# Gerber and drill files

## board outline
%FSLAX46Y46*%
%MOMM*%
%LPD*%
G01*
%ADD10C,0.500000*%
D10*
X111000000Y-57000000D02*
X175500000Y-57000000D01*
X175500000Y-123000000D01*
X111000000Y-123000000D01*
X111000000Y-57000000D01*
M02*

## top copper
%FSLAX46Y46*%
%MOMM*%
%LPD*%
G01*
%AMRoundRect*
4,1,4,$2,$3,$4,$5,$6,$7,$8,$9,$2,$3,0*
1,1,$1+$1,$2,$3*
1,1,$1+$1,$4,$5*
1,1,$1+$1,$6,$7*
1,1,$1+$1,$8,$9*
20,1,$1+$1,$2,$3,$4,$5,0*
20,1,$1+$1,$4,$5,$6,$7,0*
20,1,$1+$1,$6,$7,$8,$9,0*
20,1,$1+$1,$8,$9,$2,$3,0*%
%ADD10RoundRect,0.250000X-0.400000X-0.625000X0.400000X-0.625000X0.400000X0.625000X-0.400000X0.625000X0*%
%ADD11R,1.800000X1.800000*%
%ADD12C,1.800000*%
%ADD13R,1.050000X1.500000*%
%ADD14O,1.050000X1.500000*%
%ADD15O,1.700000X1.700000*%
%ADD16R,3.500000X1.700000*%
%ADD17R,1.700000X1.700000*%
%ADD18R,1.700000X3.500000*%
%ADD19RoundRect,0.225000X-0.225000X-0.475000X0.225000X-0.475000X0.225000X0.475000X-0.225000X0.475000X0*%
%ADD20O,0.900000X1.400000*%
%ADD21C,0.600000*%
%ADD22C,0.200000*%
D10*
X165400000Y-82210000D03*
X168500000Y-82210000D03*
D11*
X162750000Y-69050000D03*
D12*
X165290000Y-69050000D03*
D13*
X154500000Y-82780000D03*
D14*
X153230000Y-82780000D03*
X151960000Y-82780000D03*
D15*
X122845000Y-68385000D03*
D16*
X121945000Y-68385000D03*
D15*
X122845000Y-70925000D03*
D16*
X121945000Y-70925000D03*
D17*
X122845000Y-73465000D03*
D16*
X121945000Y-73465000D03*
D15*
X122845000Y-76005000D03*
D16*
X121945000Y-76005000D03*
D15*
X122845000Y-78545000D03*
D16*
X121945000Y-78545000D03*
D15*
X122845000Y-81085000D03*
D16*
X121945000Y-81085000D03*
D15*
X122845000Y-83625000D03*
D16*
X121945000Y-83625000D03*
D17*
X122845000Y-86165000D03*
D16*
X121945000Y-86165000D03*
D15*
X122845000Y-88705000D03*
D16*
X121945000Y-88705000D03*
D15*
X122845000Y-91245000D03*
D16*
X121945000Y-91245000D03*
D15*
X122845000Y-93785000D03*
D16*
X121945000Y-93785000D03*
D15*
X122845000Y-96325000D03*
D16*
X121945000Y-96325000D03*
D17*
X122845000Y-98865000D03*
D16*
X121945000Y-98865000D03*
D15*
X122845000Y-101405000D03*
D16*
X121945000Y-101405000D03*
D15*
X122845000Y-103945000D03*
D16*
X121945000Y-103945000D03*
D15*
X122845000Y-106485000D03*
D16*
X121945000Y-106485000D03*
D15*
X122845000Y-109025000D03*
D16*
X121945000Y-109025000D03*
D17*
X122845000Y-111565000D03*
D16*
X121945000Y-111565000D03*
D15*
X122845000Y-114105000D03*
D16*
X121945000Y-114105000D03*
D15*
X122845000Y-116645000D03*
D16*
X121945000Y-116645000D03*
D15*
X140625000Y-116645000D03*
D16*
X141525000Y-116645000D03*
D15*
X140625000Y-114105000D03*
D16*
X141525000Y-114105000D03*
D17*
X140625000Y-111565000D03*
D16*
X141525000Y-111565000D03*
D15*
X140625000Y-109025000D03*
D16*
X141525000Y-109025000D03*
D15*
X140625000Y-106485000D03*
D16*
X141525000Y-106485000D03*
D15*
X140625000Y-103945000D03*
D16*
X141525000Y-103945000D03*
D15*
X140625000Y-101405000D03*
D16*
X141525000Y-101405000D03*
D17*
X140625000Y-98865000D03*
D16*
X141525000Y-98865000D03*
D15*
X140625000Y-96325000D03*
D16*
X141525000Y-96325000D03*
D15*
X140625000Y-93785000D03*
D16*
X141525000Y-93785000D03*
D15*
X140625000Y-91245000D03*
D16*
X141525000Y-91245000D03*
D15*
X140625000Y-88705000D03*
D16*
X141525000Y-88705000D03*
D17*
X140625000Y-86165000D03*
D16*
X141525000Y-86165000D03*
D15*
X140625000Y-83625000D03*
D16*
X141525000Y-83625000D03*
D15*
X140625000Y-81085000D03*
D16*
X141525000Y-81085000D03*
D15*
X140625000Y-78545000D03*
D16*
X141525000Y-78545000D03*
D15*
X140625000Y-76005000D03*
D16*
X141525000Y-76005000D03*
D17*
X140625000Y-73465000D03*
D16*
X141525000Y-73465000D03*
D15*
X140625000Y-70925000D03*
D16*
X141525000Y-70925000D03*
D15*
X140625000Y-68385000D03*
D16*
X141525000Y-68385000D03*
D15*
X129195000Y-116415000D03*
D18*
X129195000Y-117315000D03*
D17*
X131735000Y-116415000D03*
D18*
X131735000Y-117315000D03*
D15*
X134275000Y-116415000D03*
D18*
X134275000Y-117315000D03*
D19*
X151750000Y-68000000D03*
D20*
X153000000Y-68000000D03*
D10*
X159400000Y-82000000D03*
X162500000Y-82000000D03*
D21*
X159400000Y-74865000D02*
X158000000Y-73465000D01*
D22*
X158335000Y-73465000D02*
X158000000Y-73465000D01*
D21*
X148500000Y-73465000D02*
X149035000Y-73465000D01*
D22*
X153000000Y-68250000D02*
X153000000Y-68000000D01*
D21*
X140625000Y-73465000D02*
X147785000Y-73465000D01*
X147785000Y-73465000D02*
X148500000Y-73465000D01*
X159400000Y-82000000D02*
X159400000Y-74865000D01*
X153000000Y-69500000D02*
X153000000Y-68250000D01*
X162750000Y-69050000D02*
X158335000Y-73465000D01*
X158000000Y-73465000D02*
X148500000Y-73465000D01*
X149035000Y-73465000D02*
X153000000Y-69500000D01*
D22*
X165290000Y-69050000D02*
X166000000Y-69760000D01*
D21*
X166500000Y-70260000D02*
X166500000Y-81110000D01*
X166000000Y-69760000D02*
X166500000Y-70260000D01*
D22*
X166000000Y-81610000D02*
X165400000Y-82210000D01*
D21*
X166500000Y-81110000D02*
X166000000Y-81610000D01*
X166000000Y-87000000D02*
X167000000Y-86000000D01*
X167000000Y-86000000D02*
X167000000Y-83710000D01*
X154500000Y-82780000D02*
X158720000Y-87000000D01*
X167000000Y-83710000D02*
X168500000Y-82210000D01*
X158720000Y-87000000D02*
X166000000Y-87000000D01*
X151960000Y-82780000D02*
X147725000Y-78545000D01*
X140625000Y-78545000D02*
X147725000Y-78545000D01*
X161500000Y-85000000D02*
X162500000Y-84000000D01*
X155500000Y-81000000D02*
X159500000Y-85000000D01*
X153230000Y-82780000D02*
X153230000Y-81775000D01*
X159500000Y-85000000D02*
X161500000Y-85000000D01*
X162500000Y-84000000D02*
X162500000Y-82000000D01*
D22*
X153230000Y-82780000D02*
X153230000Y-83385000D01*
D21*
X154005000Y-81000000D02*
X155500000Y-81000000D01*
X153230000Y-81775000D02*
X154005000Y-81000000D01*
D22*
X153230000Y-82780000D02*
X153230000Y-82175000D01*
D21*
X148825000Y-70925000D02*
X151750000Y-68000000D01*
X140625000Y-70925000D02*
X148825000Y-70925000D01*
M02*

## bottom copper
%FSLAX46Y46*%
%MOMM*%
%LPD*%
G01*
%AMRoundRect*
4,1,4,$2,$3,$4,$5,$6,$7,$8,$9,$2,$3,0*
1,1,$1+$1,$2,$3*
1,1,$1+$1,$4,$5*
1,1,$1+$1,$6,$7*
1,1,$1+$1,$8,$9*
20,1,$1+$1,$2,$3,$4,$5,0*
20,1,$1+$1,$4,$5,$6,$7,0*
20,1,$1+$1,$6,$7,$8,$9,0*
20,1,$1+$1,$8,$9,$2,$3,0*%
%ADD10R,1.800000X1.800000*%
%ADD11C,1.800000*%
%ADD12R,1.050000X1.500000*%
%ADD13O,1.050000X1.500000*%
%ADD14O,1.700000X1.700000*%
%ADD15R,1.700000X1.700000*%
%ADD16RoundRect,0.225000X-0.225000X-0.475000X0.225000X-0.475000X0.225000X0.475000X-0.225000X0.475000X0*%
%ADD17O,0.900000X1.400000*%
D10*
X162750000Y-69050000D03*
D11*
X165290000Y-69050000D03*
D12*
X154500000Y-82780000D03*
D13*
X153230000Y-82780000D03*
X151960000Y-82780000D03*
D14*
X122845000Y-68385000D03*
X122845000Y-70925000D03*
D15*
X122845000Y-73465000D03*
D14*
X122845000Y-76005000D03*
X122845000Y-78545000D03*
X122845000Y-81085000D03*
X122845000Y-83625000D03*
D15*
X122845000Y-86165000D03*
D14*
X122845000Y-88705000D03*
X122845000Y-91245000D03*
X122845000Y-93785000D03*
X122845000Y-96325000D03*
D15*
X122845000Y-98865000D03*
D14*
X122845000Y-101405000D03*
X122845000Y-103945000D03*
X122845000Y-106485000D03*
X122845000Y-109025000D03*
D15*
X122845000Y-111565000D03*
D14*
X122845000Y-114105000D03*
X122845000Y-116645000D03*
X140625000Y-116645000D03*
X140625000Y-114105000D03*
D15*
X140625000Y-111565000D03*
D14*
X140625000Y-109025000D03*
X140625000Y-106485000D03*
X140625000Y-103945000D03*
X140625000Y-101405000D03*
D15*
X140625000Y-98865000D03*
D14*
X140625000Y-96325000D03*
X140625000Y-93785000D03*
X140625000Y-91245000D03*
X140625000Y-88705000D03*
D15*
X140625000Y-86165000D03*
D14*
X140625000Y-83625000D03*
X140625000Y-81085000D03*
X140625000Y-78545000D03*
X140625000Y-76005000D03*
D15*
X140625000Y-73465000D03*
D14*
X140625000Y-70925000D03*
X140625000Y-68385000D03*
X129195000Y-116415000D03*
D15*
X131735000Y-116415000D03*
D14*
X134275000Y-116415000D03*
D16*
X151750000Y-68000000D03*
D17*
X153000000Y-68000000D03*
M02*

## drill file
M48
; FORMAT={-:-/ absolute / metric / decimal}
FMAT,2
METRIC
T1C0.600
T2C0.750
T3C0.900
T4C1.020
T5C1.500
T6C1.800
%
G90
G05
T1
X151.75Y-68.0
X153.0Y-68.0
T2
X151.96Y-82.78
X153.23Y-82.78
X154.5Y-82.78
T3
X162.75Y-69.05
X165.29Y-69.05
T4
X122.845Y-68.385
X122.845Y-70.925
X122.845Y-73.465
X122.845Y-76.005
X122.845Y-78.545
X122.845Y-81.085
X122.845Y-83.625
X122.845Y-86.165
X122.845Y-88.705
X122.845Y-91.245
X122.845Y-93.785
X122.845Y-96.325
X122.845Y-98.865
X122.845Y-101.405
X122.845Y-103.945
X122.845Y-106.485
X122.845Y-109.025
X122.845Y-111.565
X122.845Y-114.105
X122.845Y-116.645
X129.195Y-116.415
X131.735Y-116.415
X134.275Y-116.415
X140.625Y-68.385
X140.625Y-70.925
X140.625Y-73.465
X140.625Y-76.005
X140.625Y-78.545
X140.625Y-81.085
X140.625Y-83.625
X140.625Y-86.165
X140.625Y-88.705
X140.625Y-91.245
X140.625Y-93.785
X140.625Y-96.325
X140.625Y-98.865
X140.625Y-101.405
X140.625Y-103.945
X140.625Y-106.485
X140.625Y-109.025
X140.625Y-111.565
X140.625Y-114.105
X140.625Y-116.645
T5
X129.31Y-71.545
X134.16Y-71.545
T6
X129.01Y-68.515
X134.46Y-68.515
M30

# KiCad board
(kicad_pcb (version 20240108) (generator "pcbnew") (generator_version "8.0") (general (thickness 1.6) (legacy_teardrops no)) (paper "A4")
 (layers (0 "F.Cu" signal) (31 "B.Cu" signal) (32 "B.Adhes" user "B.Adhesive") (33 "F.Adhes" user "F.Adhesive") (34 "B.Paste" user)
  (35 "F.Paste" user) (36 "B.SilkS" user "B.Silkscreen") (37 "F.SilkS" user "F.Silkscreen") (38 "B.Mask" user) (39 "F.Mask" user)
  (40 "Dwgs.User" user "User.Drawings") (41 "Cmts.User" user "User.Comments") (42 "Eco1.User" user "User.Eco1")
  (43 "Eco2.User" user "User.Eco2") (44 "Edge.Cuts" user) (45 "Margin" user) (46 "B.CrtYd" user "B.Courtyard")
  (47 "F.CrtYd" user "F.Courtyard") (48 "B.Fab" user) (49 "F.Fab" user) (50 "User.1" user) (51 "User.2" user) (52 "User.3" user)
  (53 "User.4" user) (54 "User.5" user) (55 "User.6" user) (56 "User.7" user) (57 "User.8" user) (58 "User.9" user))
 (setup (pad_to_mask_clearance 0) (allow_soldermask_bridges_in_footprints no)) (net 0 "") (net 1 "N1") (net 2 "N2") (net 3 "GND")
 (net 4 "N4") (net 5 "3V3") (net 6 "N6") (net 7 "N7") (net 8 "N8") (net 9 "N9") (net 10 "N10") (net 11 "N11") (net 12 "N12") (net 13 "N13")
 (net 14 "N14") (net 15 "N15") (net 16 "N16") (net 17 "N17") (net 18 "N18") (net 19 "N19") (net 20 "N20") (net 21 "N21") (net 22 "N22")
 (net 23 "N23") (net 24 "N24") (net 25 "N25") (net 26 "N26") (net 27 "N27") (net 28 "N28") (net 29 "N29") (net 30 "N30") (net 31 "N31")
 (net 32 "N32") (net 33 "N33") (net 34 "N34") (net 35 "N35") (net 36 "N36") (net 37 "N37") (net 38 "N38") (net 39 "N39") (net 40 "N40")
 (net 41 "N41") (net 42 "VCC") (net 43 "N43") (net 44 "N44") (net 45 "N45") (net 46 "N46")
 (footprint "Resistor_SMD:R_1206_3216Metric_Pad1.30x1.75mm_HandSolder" (layer "F.Cu") (at 166.95 82.21)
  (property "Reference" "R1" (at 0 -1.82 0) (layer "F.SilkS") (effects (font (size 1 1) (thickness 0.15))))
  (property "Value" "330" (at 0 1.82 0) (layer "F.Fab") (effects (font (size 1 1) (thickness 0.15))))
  (pad "1" smd roundrect (at -1.55 0) (size 1.3 1.75) (layers "F.Cu" "F.Paste" "F.Mask") (roundrect_rratio 0.192308) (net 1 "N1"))
  (pad "2" smd roundrect (at 1.55 0) (size 1.3 1.75) (layers "F.Cu" "F.Paste" "F.Mask") (roundrect_rratio 0.192308) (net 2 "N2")))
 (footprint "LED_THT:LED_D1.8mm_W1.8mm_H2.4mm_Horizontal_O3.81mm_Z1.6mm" (layer "F.Cu") (at 162.75 69.05)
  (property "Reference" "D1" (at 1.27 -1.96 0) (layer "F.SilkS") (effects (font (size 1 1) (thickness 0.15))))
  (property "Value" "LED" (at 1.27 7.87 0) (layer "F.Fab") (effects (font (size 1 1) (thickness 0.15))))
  (pad "1" thru_hole rect (at 0 0) (size 1.8 1.8) (drill 0.9) (layers "*.Cu" "*.Mask") (remove_unused_layers no) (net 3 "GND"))
  (pad "2" thru_hole circle (at 2.54 0) (size 1.8 1.8) (drill 0.9) (layers "*.Cu" "*.Mask") (remove_unused_layers no) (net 1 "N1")))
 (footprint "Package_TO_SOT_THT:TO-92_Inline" (layer "F.Cu") (at 154.5 82.78 180)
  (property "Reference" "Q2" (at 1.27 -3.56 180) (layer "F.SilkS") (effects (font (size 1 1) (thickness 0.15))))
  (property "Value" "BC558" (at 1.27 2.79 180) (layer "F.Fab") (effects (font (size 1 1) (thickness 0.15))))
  (pad "1" thru_hole rect (at 0 0 180) (size 1.05 1.5) (drill 0.75) (layers "*.Cu" "*.Mask") (remove_unused_layers no) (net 2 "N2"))
  (pad "2" thru_hole oval (at 1.27 0 180) (size 1.05 1.5) (drill 0.75) (layers "*.Cu" "*.Mask") (remove_unused_layers no) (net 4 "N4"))
  (pad "3" thru_hole oval (at 2.54 0 180) (size 1.05 1.5) (drill 0.75) (layers "*.Cu" "*.Mask") (remove_unused_layers no) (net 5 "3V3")))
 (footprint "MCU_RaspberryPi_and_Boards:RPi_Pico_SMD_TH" (layer "F.Cu") (at 131.735 92.515)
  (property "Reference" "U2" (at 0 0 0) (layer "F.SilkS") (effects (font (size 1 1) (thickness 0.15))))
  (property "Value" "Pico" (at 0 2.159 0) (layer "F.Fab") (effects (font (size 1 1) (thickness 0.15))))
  (pad "" np_thru_hole oval (at -2.725 -24) (size 1.8 1.8) (drill 1.8) (layers "*.Cu" "*.Mask"))
  (pad "" np_thru_hole oval (at -2.425 -20.97) (size 1.5 1.5) (drill 1.5) (layers "*.Cu" "*.Mask"))
  (pad "" np_thru_hole oval (at 2.425 -20.97) (size 1.5 1.5) (drill 1.5) (layers "*.Cu" "*.Mask"))
  (pad "" np_thru_hole oval (at 2.725 -24) (size 1.8 1.8) (drill 1.8) (layers "*.Cu" "*.Mask"))
  (pad "1" thru_hole oval (at -8.89 -24.13) (size 1.7 1.7) (drill 1.02) (layers "*.Cu" "*.Mask") (remove_unused_layers no) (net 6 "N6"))
  (pad "1" smd rect (at -8.89 -24.13) (size 3.5 1.7) (drill (offset -0.9 0)) (layers "F.Cu" "F.Mask") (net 6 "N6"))
  (pad "2" thru_hole oval (at -8.89 -21.59) (size 1.7 1.7) (drill 1.02) (layers "*.Cu" "*.Mask") (remove_unused_layers no) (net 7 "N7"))
  (pad "2" smd rect (at -8.89 -21.59) (size 3.5 1.7) (drill (offset -0.9 0)) (layers "F.Cu" "F.Mask") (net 7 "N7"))
  (pad "3" thru_hole rect (at -8.89 -19.05) (size 1.7 1.7) (drill 1.02) (layers "*.Cu" "*.Mask") (remove_unused_layers no) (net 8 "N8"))
  (pad "3" smd rect (at -8.89 -19.05) (size 3.5 1.7) (drill (offset -0.9 0)) (layers "F.Cu" "F.Mask") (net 8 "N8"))
  (pad "4" thru_hole oval (at -8.89 -16.51) (size 1.7 1.7) (drill 1.02) (layers "*.Cu" "*.Mask") (remove_unused_layers no) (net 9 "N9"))
  (pad "4" smd rect (at -8.89 -16.51) (size 3.5 1.7) (drill (offset -0.9 0)) (layers "F.Cu" "F.Mask") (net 9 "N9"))
  (pad "5" thru_hole oval (at -8.89 -13.97) (size 1.7 1.7) (drill 1.02) (layers "*.Cu" "*.Mask") (remove_unused_layers no) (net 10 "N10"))
  (pad "5" smd rect (at -8.89 -13.97) (size 3.5 1.7) (drill (offset -0.9 0)) (layers "F.Cu" "F.Mask") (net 10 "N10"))
  (pad "6" thru_hole oval (at -8.89 -11.43) (size 1.7 1.7) (drill 1.02) (layers "*.Cu" "*.Mask") (remove_unused_layers no) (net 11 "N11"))
  (pad "6" smd rect (at -8.89 -11.43) (size 3.5 1.7) (drill (offset -0.9 0)) (layers "F.Cu" "F.Mask") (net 11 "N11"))
  (pad "7" thru_hole oval (at -8.89 -8.89) (size 1.7 1.7) (drill 1.02) (layers "*.Cu" "*.Mask") (remove_unused_layers no) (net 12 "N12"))
  (pad "7" smd rect (at -8.89 -8.89) (size 3.5 1.7) (drill (offset -0.9 0)) (layers "F.Cu" "F.Mask") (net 12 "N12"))
  (pad "8" thru_hole rect (at -8.89 -6.35) (size 1.7 1.7) (drill 1.02) (layers "*.Cu" "*.Mask") (remove_unused_layers no) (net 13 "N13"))
  (pad "8" smd rect (at -8.89 -6.35) (size 3.5 1.7) (drill (offset -0.9 0)) (layers "F.Cu" "F.Mask") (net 13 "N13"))
  (pad "9" thru_hole oval (at -8.89 -3.81) (size 1.7 1.7) (drill 1.02) (layers "*.Cu" "*.Mask") (remove_unused_layers no) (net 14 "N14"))
  (pad "9" smd rect (at -8.89 -3.81) (size 3.5 1.7) (drill (offset -0.9 0)) (layers "F.Cu" "F.Mask") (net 14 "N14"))
  (pad "10" thru_hole oval (at -8.89 -1.27) (size 1.7 1.7) (drill 1.02) (layers "*.Cu" "*.Mask") (remove_unused_layers no) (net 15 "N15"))
  (pad "10" smd rect (at -8.89 -1.27) (size 3.5 1.7) (drill (offset -0.9 0)) (layers "F.Cu" "F.Mask") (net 15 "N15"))
  (pad "11" thru_hole oval (at -8.89 1.27) (size 1.7 1.7) (drill 1.02) (layers "*.Cu" "*.Mask") (remove_unused_layers no) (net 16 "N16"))
  (pad "11" smd rect (at -8.89 1.27) (size 3.5 1.7) (drill (offset -0.9 0)) (layers "F.Cu" "F.Mask") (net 16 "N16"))
  (pad "12" thru_hole oval (at -8.89 3.81) (size 1.7 1.7) (drill 1.02) (layers "*.Cu" "*.Mask") (remove_unused_layers no) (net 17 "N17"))
  (pad "12" smd rect (at -8.89 3.81) (size 3.5 1.7) (drill (offset -0.9 0)) (layers "F.Cu" "F.Mask") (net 17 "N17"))
  (pad "13" thru_hole rect (at -8.89 6.35) (size 1.7 1.7) (drill 1.02) (layers "*.Cu" "*.Mask") (remove_unused_layers no) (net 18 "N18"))
  (pad "13" smd rect (at -8.89 6.35) (size 3.5 1.7) (drill (offset -0.9 0)) (layers "F.Cu" "F.Mask") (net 18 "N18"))
  (pad "14" thru_hole oval (at -8.89 8.89) (size 1.7 1.7) (drill 1.02) (layers "*.Cu" "*.Mask") (remove_unused_layers no) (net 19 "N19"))
  (pad "14" smd rect (at -8.89 8.89) (size 3.5 1.7) (drill (offset -0.9 0)) (layers "F.Cu" "F.Mask") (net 19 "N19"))
  (pad "15" thru_hole oval (at -8.89 11.43) (size 1.7 1.7) (drill 1.02) (layers "*.Cu" "*.Mask") (remove_unused_layers no) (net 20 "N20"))
  (pad "15" smd rect (at -8.89 11.43) (size 3.5 1.7) (drill (offset -0.9 0)) (layers "F.Cu" "F.Mask") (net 20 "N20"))
  (pad "16" thru_hole oval (at -8.89 13.97) (size 1.7 1.7) (drill 1.02) (layers "*.Cu" "*.Mask") (remove_unused_layers no) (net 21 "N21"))
  (pad "16" smd rect (at -8.89 13.97) (size 3.5 1.7) (drill (offset -0.9 0)) (layers "F.Cu" "F.Mask") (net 21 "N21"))
  (pad "17" thru_hole oval (at -8.89 16.51) (size 1.7 1.7) (drill 1.02) (layers "*.Cu" "*.Mask") (remove_unused_layers no) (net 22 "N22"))
  (pad "17" smd rect (at -8.89 16.51) (size 3.5 1.7) (drill (offset -0.9 0)) (layers "F.Cu" "F.Mask") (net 22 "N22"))
  (pad "18" thru_hole rect (at -8.89 19.05) (size 1.7 1.7) (drill 1.02) (layers "*.Cu" "*.Mask") (remove_unused_layers no) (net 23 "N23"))
  (pad "18" smd rect (at -8.89 19.05) (size 3.5 1.7) (drill (offset -0.9 0)) (layers "F.Cu" "F.Mask") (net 23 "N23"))
  (pad "19" thru_hole oval (at -8.89 21.59) (size 1.7 1.7) (drill 1.02) (layers "*.Cu" "*.Mask") (remove_unused_layers no) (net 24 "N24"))
  (pad "19" smd rect (at -8.89 21.59) (size 3.5 1.7) (drill (offset -0.9 0)) (layers "F.Cu" "F.Mask") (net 24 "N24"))
  (pad "20" thru_hole oval (at -8.89 24.13) (size 1.7 1.7) (drill 1.02) (layers "*.Cu" "*.Mask") (remove_unused_layers no) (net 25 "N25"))
  (pad "20" smd rect (at -8.89 24.13) (size 3.5 1.7) (drill (offset -0.9 0)) (layers "F.Cu" "F.Mask") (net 25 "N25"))
  (pad "21" thru_hole oval (at 8.89 24.13) (size 1.7 1.7) (drill 1.02) (layers "*.Cu" "*.Mask") (remove_unused_layers no) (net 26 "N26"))
  (pad "21" smd rect (at 8.89 24.13) (size 3.5 1.7) (drill (offset 0.9 0)) (layers "F.Cu" "F.Mask") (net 26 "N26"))
  (pad "22" thru_hole oval (at 8.89 21.59) (size 1.7 1.7) (drill 1.02) (layers "*.Cu" "*.Mask") (remove_unused_layers no) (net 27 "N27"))
  (pad "22" smd rect (at 8.89 21.59) (size 3.5 1.7) (drill (offset 0.9 0)) (layers "F.Cu" "F.Mask") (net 27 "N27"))
  (pad "23" thru_hole rect (at 8.89 19.05) (size 1.7 1.7) (drill 1.02) (layers "*.Cu" "*.Mask") (remove_unused_layers no) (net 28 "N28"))
  (pad "23" smd rect (at 8.89 19.05) (size 3.5 1.7) (drill (offset 0.9 0)) (layers "F.Cu" "F.Mask") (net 28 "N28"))
  (pad "24" thru_hole oval (at 8.89 16.51) (size 1.7 1.7) (drill 1.02) (layers "*.Cu" "*.Mask") (remove_unused_layers no) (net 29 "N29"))
  (pad "24" smd rect (at 8.89 16.51) (size 3.5 1.7) (drill (offset 0.9 0)) (layers "F.Cu" "F.Mask") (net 29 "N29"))
  (pad "25" thru_hole oval (at 8.89 13.97) (size 1.7 1.7) (drill 1.02) (layers "*.Cu" "*.Mask") (remove_unused_layers no) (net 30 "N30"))
  (pad "25" smd rect (at 8.89 13.97) (size 3.5 1.7) (drill (offset 0.9 0)) (layers "F.Cu" "F.Mask") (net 30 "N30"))
  (pad "26" thru_hole oval (at 8.89 11.43) (size 1.7 1.7) (drill 1.02) (layers "*.Cu" "*.Mask") (remove_unused_layers no) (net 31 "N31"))
  (pad "26" smd rect (at 8.89 11.43) (size 3.5 1.7) (drill (offset 0.9 0)) (layers "F.Cu" "F.Mask") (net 31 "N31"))
  (pad "27" thru_hole oval (at 8.89 8.89) (size 1.7 1.7) (drill 1.02) (layers "*.Cu" "*.Mask") (remove_unused_layers no) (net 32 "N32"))
  (pad "27" smd rect (at 8.89 8.89) (size 3.5 1.7) (drill (offset 0.9 0)) (layers "F.Cu" "F.Mask") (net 32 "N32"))
  (pad "28" thru_hole rect (at 8.89 6.35) (size 1.7 1.7) (drill 1.02) (layers "*.Cu" "*.Mask") (remove_unused_layers no) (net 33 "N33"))
  (pad "28" smd rect (at 8.89 6.35) (size 3.5 1.7) (drill (offset 0.9 0)) (layers "F.Cu" "F.Mask") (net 33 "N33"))
  (pad "29" thru_hole oval (at 8.89 3.81) (size 1.7 1.7) (drill 1.02) (layers "*.Cu" "*.Mask") (remove_unused_layers no) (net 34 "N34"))
  (pad "29" smd rect (at 8.89 3.81) (size 3.5 1.7) (drill (offset 0.9 0)) (layers "F.Cu" "F.Mask") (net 34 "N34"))
  (pad "30" thru_hole oval (at 8.89 1.27) (size 1.7 1.7) (drill 1.02) (layers "*.Cu" "*.Mask") (remove_unused_layers no) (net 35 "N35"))
  (pad "30" smd rect (at 8.89 1.27) (size 3.5 1.7) (drill (offset 0.9 0)) (layers "F.Cu" "F.Mask") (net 35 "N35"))
  (pad "31" thru_hole oval (at 8.89 -1.27) (size 1.7 1.7) (drill 1.02) (layers "*.Cu" "*.Mask") (remove_unused_layers no) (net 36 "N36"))
  (pad "31" smd rect (at 8.89 -1.27) (size 3.5 1.7) (drill (offset 0.9 0)) (layers "F.Cu" "F.Mask") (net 36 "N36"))
  (pad "32" thru_hole oval (at 8.89 -3.81) (size 1.7 1.7) (drill 1.02) (layers "*.Cu" "*.Mask") (remove_unused_layers no) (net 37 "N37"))
  (pad "32" smd rect (at 8.89 -3.81) (size 3.5 1.7) (drill (offset 0.9 0)) (layers "F.Cu" "F.Mask") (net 37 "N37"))
  (pad "33" thru_hole rect (at 8.89 -6.35) (size 1.7 1.7) (drill 1.02) (layers "*.Cu" "*.Mask") (remove_unused_layers no) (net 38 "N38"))
  (pad "33" smd rect (at 8.89 -6.35) (size 3.5 1.7) (drill (offset 0.9 0)) (layers "F.Cu" "F.Mask") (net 38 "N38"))
  (pad "34" thru_hole oval (at 8.89 -8.89) (size 1.7 1.7) (drill 1.02) (layers "*.Cu" "*.Mask") (remove_unused_layers no) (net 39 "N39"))
  (pad "34" smd rect (at 8.89 -8.89) (size 3.5 1.7) (drill (offset 0.9 0)) (layers "F.Cu" "F.Mask") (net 39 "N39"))
  (pad "35" thru_hole oval (at 8.89 -11.43) (size 1.7 1.7) (drill 1.02) (layers "*.Cu" "*.Mask") (remove_unused_layers no) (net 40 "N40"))
  (pad "35" smd rect (at 8.89 -11.43) (size 3.5 1.7) (drill (offset 0.9 0)) (layers "F.Cu" "F.Mask") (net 40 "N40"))
  (pad "36" thru_hole oval (at 8.89 -13.97) (size 1.7 1.7) (drill 1.02) (layers "*.Cu" "*.Mask") (remove_unused_layers no) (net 5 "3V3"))
  (pad "36" smd rect (at 8.89 -13.97) (size 3.5 1.7) (drill (offset 0.9 0)) (layers "F.Cu" "F.Mask") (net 5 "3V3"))
  (pad "37" thru_hole oval (at 8.89 -16.51) (size 1.7 1.7) (drill 1.02) (layers "*.Cu" "*.Mask") (remove_unused_layers no) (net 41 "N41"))
  (pad "37" smd rect (at 8.89 -16.51) (size 3.5 1.7) (drill (offset 0.9 0)) (layers "F.Cu" "F.Mask") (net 41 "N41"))
  (pad "38" thru_hole rect (at 8.89 -19.05) (size 1.7 1.7) (drill 1.02) (layers "*.Cu" "*.Mask") (remove_unused_layers no) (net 3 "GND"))
  (pad "38" smd rect (at 8.89 -19.05) (size 3.5 1.7) (drill (offset 0.9 0)) (layers "F.Cu" "F.Mask") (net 3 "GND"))
  (pad "39" thru_hole oval (at 8.89 -21.59) (size 1.7 1.7) (drill 1.02) (layers "*.Cu" "*.Mask") (remove_unused_layers no) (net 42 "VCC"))
  (pad "39" smd rect (at 8.89 -21.59) (size 3.5 1.7) (drill (offset 0.9 0)) (layers "F.Cu" "F.Mask") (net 42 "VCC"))
  (pad "40" thru_hole oval (at 8.89 -24.13) (size 1.7 1.7) (drill 1.02) (layers "*.Cu" "*.Mask") (remove_unused_layers no) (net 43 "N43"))
  (pad "40" smd rect (at 8.89 -24.13) (size 3.5 1.7) (drill (offset 0.9 0)) (layers "F.Cu" "F.Mask") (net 43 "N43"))
  (pad "41" thru_hole oval (at -2.54 23.9) (size 1.7 1.7) (drill 1.02) (layers "*.Cu" "*.Mask") (remove_unused_layers no) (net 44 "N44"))
  (pad "41" smd rect (at -2.54 23.9 90) (size 3.5 1.7) (drill (offset -0.9 0)) (layers "F.Cu" "F.Mask") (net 44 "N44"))
  (pad "42" thru_hole rect (at 0 23.9) (size 1.7 1.7) (drill 1.02) (layers "*.Cu" "*.Mask") (remove_unused_layers no) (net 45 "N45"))
  (pad "42" smd rect (at 0 23.9 90) (size 3.5 1.7) (drill (offset -0.9 0)) (layers "F.Cu" "F.Mask") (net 45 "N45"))
  (pad "43" thru_hole oval (at 2.54 23.9) (size 1.7 1.7) (drill 1.02) (layers "*.Cu" "*.Mask") (remove_unused_layers no) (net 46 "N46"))
  (pad "43" smd rect (at 2.54 23.9 90) (size 3.5 1.7) (drill (offset -0.9 0)) (layers "F.Cu" "F.Mask") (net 46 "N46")))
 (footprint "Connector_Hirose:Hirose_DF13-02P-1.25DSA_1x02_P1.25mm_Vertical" (layer "F.Cu") (at 151.75 68)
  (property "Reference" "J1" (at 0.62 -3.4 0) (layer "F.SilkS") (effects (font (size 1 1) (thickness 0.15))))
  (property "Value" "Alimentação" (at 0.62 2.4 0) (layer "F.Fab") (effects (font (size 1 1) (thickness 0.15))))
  (pad "1" thru_hole roundrect (at 0 0) (size 0.9 1.4) (drill 0.6) (layers "*.Cu" "*.Mask") (remove_unused_layers no)
   (roundrect_rratio 0.25) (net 42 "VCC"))
  (pad "2" thru_hole oval (at 1.25 0) (size 0.9 1.4) (drill 0.6) (layers "*.Cu" "*.Mask") (remove_unused_layers no) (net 3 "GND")))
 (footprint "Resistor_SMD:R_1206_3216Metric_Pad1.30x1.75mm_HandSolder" (layer "F.Cu") (at 160.95 82)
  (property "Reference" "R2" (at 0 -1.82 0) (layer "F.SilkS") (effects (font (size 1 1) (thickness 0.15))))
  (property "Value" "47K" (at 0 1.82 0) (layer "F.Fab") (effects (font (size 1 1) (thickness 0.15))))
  (pad "1" smd roundrect (at -1.55 0) (size 1.3 1.75) (layers "F.Cu" "F.Paste" "F.Mask") (roundrect_rratio 0.192308) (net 3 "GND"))
  (pad "2" smd roundrect (at 1.55 0) (size 1.3 1.75) (layers "F.Cu" "F.Paste" "F.Mask") (roundrect_rratio 0.192308) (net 4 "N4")))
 (gr_rect (start 111 57) (end 175.5 123) (stroke (width 0.5) (type default)) (fill none) (layer "Edge.Cuts"))
 (segment (start 159.4 74.865) (end 158 73.465) (width 0.6) (layer "F.Cu") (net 3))
 (segment (start 158.335 73.465) (end 158 73.465) (width 0.2) (layer "F.Cu") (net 3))
 (segment (start 148.5 73.465) (end 149.035 73.465) (width 0.6) (layer "F.Cu") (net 3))
 (segment (start 153 68.25) (end 153 68) (width 0.2) (layer "F.Cu") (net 3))
 (segment (start 140.625 73.465) (end 147.785 73.465) (width 0.6) (layer "F.Cu") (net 3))
 (segment (start 147.785 73.465) (end 148.5 73.465) (width 0.6) (layer "F.Cu") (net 3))
 (segment (start 159.4 82) (end 159.4 74.865) (width 0.6) (layer "F.Cu") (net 3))
 (segment (start 153 69.5) (end 153 68.25) (width 0.6) (layer "F.Cu") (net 3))
 (segment (start 162.75 69.05) (end 158.335 73.465) (width 0.6) (layer "F.Cu") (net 3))
 (segment (start 158 73.465) (end 148.5 73.465) (width 0.6) (layer "F.Cu") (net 3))
 (segment (start 149.035 73.465) (end 153 69.5) (width 0.6) (layer "F.Cu") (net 3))
 (segment (start 165.29 69.05) (end 166 69.76) (width 0.2) (layer "F.Cu") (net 1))
 (segment (start 166.5 70.26) (end 166.5 81.11) (width 0.6) (layer "F.Cu") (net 1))
 (segment (start 166 69.76) (end 166.5 70.26) (width 0.6) (layer "F.Cu") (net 1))
 (segment (start 166 81.61) (end 165.4 82.21) (width 0.2) (layer "F.Cu") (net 1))
 (segment (start 166.5 81.11) (end 166 81.61) (width 0.6) (layer "F.Cu") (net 1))
 (segment (start 166 87) (end 167 86) (width 0.6) (layer "F.Cu") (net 2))
 (segment (start 167 86) (end 167 83.71) (width 0.6) (layer "F.Cu") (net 2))
 (segment (start 154.5 82.78) (end 158.72 87) (width 0.6) (layer "F.Cu") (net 2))
 (segment (start 167 83.71) (end 168.5 82.21) (width 0.6) (layer "F.Cu") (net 2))
 (segment (start 158.72 87) (end 166 87) (width 0.6) (layer "F.Cu") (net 2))
 (segment (start 151.96 82.78) (end 147.725 78.545) (width 0.6) (layer "F.Cu") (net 5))
 (segment (start 140.625 78.545) (end 147.725 78.545) (width 0.6) (layer "F.Cu") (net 5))
 (segment (start 161.5 85) (end 162.5 84) (width 0.6) (layer "F.Cu") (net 4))
 (segment (start 155.5 81) (end 159.5 85) (width 0.6) (layer "F.Cu") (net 4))
 (segment (start 153.23 82.78) (end 153.23 81.775) (width 0.6) (layer "F.Cu") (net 4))
 (segment (start 159.5 85) (end 161.5 85) (width 0.6) (layer "F.Cu") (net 4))
 (segment (start 162.5 84) (end 162.5 82) (width 0.6) (layer "F.Cu") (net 4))
 (segment (start 153.23 82.78) (end 153.23 83.385) (width 0.2) (layer "F.Cu") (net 4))
 (segment (start 154.005 81) (end 155.5 81) (width 0.6) (layer "F.Cu") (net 4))
 (segment (start 153.23 81.775) (end 154.005 81) (width 0.6) (layer "F.Cu") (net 4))
 (segment (start 153.23 82.78) (end 153.23 82.175) (width 0.2) (layer "F.Cu") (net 4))
 (segment (start 148.825 70.925) (end 151.75 68) (width 0.6) (layer "F.Cu") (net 42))
 (segment (start 140.625 70.925) (end 148.825 70.925) (width 0.6) (layer "F.Cu") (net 42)))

